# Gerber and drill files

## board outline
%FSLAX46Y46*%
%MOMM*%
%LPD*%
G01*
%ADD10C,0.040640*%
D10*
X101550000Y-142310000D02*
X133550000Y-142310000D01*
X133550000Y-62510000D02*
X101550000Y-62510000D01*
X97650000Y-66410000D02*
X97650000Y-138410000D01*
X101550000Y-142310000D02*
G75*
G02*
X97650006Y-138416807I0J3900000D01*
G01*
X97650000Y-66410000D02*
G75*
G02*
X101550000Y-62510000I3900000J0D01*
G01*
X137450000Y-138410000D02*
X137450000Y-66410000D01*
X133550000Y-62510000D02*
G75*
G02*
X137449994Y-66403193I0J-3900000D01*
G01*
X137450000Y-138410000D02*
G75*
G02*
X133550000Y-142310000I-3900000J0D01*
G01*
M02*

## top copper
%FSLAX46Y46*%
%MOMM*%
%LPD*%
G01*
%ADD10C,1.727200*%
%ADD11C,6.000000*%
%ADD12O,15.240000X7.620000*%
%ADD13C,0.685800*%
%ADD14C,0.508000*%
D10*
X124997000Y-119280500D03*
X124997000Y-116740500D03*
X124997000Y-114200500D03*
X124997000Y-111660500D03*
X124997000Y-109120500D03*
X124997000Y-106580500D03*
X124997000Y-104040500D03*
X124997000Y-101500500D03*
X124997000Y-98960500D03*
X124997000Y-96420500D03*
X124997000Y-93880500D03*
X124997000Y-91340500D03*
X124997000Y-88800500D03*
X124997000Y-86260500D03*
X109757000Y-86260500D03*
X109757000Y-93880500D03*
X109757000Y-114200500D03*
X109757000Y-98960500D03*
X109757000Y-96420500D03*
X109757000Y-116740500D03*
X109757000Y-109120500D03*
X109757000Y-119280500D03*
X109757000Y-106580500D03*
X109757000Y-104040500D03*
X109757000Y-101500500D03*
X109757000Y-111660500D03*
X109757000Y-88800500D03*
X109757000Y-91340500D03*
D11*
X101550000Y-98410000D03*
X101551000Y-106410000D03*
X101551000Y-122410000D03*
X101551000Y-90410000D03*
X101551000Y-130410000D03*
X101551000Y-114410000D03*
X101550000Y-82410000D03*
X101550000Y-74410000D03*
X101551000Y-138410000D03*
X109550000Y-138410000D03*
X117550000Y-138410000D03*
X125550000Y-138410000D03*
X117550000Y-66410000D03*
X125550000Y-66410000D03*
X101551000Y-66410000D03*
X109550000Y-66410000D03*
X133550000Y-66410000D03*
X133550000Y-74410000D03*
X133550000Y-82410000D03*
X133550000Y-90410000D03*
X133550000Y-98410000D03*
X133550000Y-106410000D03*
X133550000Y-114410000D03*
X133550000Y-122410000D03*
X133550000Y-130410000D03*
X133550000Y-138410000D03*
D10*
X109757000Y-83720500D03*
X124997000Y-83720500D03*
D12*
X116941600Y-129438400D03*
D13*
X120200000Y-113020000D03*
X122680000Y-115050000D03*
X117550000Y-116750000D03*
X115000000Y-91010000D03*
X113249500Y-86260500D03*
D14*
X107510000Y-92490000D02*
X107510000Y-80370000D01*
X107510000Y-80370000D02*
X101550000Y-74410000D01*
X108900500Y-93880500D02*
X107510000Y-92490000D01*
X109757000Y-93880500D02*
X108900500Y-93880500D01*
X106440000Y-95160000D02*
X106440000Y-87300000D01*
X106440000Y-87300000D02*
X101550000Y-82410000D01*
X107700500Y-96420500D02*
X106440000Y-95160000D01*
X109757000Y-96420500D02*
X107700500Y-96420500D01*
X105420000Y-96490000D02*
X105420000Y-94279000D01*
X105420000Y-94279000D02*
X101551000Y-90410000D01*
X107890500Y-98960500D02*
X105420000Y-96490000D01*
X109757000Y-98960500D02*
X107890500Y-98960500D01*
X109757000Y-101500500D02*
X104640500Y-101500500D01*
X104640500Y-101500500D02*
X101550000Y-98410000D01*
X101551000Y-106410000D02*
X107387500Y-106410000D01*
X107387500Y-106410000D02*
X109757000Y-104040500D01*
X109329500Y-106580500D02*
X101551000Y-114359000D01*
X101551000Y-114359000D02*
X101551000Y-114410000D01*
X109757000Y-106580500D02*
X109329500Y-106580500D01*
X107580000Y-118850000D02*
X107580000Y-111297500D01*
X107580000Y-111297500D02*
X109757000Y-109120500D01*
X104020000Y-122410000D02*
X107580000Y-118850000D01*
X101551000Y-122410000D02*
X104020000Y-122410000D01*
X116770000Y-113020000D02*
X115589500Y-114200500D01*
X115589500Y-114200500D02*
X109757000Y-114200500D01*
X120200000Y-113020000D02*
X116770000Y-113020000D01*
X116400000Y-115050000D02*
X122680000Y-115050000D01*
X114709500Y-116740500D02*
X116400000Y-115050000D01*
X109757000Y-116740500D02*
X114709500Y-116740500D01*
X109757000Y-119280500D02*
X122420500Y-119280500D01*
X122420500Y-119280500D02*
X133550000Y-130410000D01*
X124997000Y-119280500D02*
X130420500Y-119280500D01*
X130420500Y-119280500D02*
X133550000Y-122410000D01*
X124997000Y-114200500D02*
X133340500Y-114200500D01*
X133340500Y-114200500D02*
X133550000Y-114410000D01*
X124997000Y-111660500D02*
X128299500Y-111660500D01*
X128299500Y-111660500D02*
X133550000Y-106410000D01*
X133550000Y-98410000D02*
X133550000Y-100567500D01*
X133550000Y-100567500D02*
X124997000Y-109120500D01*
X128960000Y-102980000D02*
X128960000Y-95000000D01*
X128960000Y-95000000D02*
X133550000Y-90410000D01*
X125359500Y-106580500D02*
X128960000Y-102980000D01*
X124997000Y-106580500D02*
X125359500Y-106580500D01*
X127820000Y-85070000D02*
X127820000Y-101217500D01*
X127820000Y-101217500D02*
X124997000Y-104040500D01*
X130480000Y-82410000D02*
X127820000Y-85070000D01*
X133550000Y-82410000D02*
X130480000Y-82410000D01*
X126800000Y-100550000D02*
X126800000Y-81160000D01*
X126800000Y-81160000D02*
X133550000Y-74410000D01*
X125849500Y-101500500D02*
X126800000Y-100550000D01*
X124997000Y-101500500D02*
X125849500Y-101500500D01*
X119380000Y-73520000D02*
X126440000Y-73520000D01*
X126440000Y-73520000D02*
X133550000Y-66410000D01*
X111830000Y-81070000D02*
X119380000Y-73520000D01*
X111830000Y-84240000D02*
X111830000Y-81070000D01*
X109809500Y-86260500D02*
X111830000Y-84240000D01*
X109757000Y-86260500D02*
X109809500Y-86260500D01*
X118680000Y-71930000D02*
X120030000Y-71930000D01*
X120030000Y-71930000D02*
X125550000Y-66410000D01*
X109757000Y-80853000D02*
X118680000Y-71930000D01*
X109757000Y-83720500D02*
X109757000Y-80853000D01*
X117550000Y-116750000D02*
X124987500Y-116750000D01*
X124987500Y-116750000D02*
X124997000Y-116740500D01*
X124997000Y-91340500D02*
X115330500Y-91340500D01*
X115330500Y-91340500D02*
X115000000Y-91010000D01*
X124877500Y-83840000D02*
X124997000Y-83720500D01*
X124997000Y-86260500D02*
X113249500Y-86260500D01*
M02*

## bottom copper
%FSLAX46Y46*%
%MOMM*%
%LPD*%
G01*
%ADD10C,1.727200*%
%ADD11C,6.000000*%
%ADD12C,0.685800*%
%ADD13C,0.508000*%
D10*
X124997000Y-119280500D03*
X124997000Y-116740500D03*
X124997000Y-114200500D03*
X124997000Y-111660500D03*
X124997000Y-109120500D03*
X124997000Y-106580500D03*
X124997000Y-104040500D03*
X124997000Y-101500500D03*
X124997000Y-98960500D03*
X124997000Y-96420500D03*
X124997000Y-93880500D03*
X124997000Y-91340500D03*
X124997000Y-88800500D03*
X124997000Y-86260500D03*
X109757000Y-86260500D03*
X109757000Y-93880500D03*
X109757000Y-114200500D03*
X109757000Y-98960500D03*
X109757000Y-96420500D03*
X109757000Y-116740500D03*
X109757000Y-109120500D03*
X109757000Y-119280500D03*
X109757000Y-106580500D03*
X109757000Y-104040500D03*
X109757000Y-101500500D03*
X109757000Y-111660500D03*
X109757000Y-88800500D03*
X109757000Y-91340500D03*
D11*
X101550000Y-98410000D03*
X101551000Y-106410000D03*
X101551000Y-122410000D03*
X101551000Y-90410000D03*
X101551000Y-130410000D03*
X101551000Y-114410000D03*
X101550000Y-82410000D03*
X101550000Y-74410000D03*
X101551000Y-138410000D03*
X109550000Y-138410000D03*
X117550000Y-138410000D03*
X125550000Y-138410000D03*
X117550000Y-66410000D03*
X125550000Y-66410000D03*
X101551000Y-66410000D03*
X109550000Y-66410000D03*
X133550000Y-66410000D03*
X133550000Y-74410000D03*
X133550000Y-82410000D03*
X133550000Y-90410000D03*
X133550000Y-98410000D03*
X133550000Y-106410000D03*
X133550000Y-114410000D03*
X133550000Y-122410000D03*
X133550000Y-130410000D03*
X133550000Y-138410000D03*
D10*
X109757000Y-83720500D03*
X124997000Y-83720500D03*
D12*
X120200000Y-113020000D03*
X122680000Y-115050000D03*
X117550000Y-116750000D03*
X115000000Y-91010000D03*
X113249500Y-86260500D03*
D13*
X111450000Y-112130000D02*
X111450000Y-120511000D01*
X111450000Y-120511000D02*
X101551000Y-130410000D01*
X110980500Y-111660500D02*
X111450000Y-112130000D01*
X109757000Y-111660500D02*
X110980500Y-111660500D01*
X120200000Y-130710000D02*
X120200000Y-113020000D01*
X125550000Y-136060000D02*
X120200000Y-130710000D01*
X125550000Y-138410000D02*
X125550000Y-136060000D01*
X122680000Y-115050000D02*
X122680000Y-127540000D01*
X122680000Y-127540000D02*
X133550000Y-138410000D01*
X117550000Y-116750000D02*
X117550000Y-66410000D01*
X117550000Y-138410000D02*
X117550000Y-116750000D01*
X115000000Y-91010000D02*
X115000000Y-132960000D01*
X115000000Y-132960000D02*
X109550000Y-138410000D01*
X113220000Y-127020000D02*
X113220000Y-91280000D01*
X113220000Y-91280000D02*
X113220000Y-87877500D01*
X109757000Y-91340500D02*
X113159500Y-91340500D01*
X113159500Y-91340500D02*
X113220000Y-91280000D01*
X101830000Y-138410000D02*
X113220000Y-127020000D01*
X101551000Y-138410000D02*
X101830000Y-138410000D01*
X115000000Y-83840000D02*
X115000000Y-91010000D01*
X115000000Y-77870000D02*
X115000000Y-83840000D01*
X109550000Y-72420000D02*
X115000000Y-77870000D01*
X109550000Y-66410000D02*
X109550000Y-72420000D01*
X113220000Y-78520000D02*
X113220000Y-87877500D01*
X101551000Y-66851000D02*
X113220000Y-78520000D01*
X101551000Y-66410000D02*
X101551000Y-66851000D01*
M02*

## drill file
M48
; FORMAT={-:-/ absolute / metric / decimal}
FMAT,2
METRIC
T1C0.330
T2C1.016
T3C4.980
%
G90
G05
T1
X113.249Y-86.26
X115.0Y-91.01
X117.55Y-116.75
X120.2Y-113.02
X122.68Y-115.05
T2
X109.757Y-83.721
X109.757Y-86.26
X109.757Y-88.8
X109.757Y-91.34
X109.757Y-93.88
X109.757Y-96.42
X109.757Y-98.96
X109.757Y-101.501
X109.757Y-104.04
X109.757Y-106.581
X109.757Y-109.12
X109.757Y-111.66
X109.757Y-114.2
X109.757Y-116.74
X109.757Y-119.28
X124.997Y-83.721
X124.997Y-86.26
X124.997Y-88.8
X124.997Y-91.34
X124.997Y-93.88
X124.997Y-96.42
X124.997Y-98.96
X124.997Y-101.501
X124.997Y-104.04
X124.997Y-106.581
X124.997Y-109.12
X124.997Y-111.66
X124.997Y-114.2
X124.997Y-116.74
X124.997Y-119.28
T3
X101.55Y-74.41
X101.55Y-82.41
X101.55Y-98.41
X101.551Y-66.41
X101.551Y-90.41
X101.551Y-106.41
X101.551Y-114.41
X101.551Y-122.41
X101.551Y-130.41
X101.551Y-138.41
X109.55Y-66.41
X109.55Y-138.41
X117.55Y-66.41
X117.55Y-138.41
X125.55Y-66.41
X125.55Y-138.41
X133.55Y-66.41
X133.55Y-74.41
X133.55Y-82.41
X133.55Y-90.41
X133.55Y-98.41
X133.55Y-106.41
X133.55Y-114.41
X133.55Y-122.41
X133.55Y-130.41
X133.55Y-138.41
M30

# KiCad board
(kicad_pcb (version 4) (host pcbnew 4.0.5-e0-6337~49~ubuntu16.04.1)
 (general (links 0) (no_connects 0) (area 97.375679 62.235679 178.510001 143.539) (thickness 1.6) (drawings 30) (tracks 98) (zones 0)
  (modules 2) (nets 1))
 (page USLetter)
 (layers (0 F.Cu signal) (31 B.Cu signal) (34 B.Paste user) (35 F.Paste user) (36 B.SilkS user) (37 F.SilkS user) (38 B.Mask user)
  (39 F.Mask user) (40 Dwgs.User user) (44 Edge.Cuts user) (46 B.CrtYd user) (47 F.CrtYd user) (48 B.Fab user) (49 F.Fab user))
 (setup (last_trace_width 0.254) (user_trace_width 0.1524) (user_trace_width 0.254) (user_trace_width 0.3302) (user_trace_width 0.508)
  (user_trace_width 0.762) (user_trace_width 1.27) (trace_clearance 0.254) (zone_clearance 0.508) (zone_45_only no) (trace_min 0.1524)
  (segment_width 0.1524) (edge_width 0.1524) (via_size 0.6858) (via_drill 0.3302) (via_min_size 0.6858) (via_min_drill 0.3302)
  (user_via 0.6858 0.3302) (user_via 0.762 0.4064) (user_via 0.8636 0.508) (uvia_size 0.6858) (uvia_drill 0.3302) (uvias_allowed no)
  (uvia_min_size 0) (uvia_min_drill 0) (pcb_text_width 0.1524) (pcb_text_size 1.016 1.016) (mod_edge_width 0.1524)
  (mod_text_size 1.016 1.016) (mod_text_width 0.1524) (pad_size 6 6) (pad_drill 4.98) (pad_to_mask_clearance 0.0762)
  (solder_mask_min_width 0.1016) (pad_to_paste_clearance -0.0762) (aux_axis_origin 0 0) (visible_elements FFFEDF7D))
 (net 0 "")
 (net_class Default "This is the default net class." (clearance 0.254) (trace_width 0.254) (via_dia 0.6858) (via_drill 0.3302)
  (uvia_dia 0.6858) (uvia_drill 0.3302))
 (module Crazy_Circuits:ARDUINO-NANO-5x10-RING (layer F.Cu) (at 101.55 90.41)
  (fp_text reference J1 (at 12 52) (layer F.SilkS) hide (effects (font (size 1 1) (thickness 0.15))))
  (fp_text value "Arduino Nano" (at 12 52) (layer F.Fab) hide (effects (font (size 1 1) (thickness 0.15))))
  (fp_line (start 0 51.9) (end 32 51.9) (layer Edge.Cuts) (width 0.04064))
  (fp_line (start 32 -27.9) (end 0 -27.9) (layer Edge.Cuts) (width 0.04064))
  (fp_line (start -3.9 -24) (end -3.9 48) (layer Edge.Cuts) (width 0.04064))
  (fp_arc (start 0 48) (end 0 51.9) (angle 89.9) (layer Edge.Cuts) (width 0.04064))
  (fp_arc (start 0 -24) (end -3.9 -24) (angle 90) (layer Edge.Cuts) (width 0.04064))
  (fp_line (start 35.9 48) (end 35.9 -24) (layer Edge.Cuts) (width 0.04064))
  (fp_arc (start 32 -24) (end 32 -27.9) (angle 89.9) (layer Edge.Cuts) (width 0.04064))
  (fp_arc (start 32 48) (end 35.9 48) (angle 90) (layer Edge.Cuts) (width 0.04064))
  (pad D13 thru_hole circle (at 23.447 28.8705 180) (size 1.7272 1.7272) (drill 1.016) (layers *.Cu *.Mask F.SilkS))
  (pad 3V3 thru_hole circle (at 23.447 26.3305 180) (size 1.7272 1.7272) (drill 1.016) (layers *.Cu *.Mask F.SilkS))
  (pad REF thru_hole circle (at 23.447 23.7905 180) (size 1.7272 1.7272) (drill 1.016) (layers *.Cu *.Mask F.SilkS))
  (pad A0 thru_hole circle (at 23.447 21.2505 180) (size 1.7272 1.7272) (drill 1.016) (layers *.Cu *.Mask F.SilkS))
  (pad A1 thru_hole circle (at 23.447 18.7105 180) (size 1.7272 1.7272) (drill 1.016) (layers *.Cu *.Mask F.SilkS))
  (pad A2 thru_hole circle (at 23.447 16.1705 180) (size 1.7272 1.7272) (drill 1.016) (layers *.Cu *.Mask F.SilkS))
  (pad A3 thru_hole circle (at 23.447 13.6305 180) (size 1.7272 1.7272) (drill 1.016) (layers *.Cu *.Mask F.SilkS))
  (pad A4 thru_hole circle (at 23.447 11.0905 180) (size 1.7272 1.7272) (drill 1.016) (layers *.Cu *.Mask F.SilkS))
  (pad A5 thru_hole circle (at 23.447 8.5505 180) (size 1.7272 1.7272) (drill 1.016) (layers *.Cu *.Mask F.SilkS))
  (pad A6 thru_hole circle (at 23.447 6.0105 180) (size 1.7272 1.7272) (drill 1.016) (layers *.Cu *.Mask F.SilkS))
  (pad A7 thru_hole circle (at 23.447 3.4705 180) (size 1.7272 1.7272) (drill 1.016) (layers *.Cu *.Mask F.SilkS))
  (pad 5V thru_hole circle (at 23.447 0.9305 180) (size 1.7272 1.7272) (drill 1.016) (layers *.Cu *.Mask F.SilkS))
  (pad RST thru_hole circle (at 23.447 -1.6095 180) (size 1.7272 1.7272) (drill 1.016) (layers *.Cu *.Mask F.SilkS))
  (pad GND thru_hole circle (at 23.447 -4.1495 180) (size 1.7272 1.7272) (drill 1.016) (layers *.Cu *.Mask F.SilkS))
  (pad D0RX thru_hole circle (at 8.207 -4.1495 180) (size 1.7272 1.7272) (drill 1.016) (layers *.Cu *.Mask F.SilkS))
  (pad D2 thru_hole circle (at 8.207 3.4705 180) (size 1.7272 1.7272) (drill 1.016) (layers *.Cu *.Mask F.SilkS))
  (pad D10 thru_hole circle (at 8.207 23.7905 180) (size 1.7272 1.7272) (drill 1.016) (layers *.Cu *.Mask F.SilkS))
  (pad D4 thru_hole circle (at 8.207 8.5505 180) (size 1.7272 1.7272) (drill 1.016) (layers *.Cu *.Mask F.SilkS))
  (pad D3 thru_hole circle (at 8.207 6.0105 180) (size 1.7272 1.7272) (drill 1.016) (layers *.Cu *.Mask F.SilkS))
  (pad D11 thru_hole circle (at 8.207 26.3305 180) (size 1.7272 1.7272) (drill 1.016) (layers *.Cu *.Mask F.SilkS))
  (pad D8 thru_hole circle (at 8.207 18.7105 180) (size 1.7272 1.7272) (drill 1.016) (layers *.Cu *.Mask F.SilkS))
  (pad D12 thru_hole circle (at 8.207 28.8705 180) (size 1.7272 1.7272) (drill 1.016) (layers *.Cu *.Mask F.SilkS))
  (pad D7 thru_hole circle (at 8.207 16.1705 180) (size 1.7272 1.7272) (drill 1.016) (layers *.Cu *.Mask F.SilkS))
  (pad D6 thru_hole circle (at 8.207 13.6305 180) (size 1.7272 1.7272) (drill 1.016) (layers *.Cu *.Mask F.SilkS))
  (pad D5 thru_hole circle (at 8.207 11.0905 180) (size 1.7272 1.7272) (drill 1.016) (layers *.Cu *.Mask F.SilkS))
  (pad D9 thru_hole circle (at 8.207 21.2505 180) (size 1.7272 1.7272) (drill 1.016) (layers *.Cu *.Mask F.SilkS))
  (pad RST thru_hole circle (at 8.207 -1.6095 180) (size 1.7272 1.7272) (drill 1.016) (layers *.Cu *.Mask F.SilkS))
  (pad GND thru_hole circle (at 8.207 0.9305 180) (size 1.7272 1.7272) (drill 1.016) (layers *.Cu *.Mask F.SilkS))
  (pad D5 thru_hole circle (at 0 8 90) (size 6 6) (drill 4.98) (layers *.Cu *.Mask))
  (pad D6 thru_hole circle (at 0.001 16 90) (size 6 6) (drill 4.98) (layers *.Cu *.Mask))
  (pad D8 thru_hole circle (at 0.001 32 90) (size 6 6) (drill 4.98) (layers *.Cu *.Mask))
  (pad D4 thru_hole circle (at 0.001 0 90) (size 6 6) (drill 4.98) (layers *.Cu *.Mask))
  (pad D9 thru_hole circle (at 0.001 40 90) (size 6 6) (drill 4.98) (layers *.Cu *.Mask))
  (pad D7 thru_hole circle (at 0.001 24 90) (size 6 6) (drill 4.98) (layers *.Cu *.Mask))
  (pad D3 thru_hole circle (at 0 -8 90) (size 6 6) (drill 4.98) (layers *.Cu *.Mask))
  (pad D2 thru_hole circle (at 0 -16 90) (size 6 6) (drill 4.98) (layers *.Cu *.Mask))
  (pad GND thru_hole circle (at 0.001 48 90) (size 6 6) (drill 4.98) (layers *.Cu *.Mask))
  (pad 5V thru_hole circle (at 8 48 90) (size 6 6) (drill 4.98) (layers *.Cu *.Mask))
  (pad 3.3V thru_hole circle (at 16 48 90) (size 6 6) (drill 4.98) (layers *.Cu *.Mask))
  (pad D10 thru_hole circle (at 24 48 90) (size 6 6) (drill 4.98) (layers *.Cu *.Mask))
  (pad 3.3V thru_hole circle (at 16 -24 90) (size 6 6) (drill 4.98) (layers *.Cu *.Mask))
  (pad D1TX thru_hole circle (at 24 -24 90) (size 6 6) (drill 4.98) (layers *.Cu *.Mask))
  (pad GND thru_hole circle (at 0.001 -24 90) (size 6 6) (drill 4.98) (layers *.Cu *.Mask))
  (pad 5V thru_hole circle (at 8 -24 90) (size 6 6) (drill 4.98) (layers *.Cu *.Mask))
  (pad D0RX thru_hole circle (at 32 -24 90) (size 6 6) (drill 4.98) (layers *.Cu *.Mask))
  (pad A4 thru_hole circle (at 32 -16 90) (size 6 6) (drill 4.98) (layers *.Cu *.Mask))
  (pad A3 thru_hole circle (at 32 -8 90) (size 6 6) (drill 4.98) (layers *.Cu *.Mask))
  (pad A2 thru_hole circle (at 32 0 90) (size 6 6) (drill 4.98) (layers *.Cu *.Mask))
  (pad A1 thru_hole circle (at 32 8 90) (size 6 6) (drill 4.98) (layers *.Cu *.Mask))
  (pad A0 thru_hole circle (at 32 16 90) (size 6 6) (drill 4.98) (layers *.Cu *.Mask))
  (pad AREF thru_hole circle (at 32 24 90) (size 6 6) (drill 4.98) (layers *.Cu *.Mask))
  (pad D13 thru_hole circle (at 32 32 90) (size 6 6) (drill 4.98) (layers *.Cu *.Mask))
  (pad D12 thru_hole circle (at 32 40 90) (size 6 6) (drill 4.98) (layers *.Cu *.Mask))
  (pad D11 thru_hole circle (at 32 48 90) (size 6 6) (drill 4.98) (layers *.Cu *.Mask))
  (pad D1TX thru_hole circle (at 8.207 -6.6895 180) (size 1.7272 1.7272) (drill 1.016) (layers *.Cu *.Mask F.SilkS))
  (pad VIN thru_hole circle (at 23.447 -6.6895 180) (size 1.7272 1.7272) (drill 1.016) (layers *.Cu *.Mask F.SilkS)))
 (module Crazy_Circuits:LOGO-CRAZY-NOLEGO (layer F.Cu) (at 116.9416 133.3754)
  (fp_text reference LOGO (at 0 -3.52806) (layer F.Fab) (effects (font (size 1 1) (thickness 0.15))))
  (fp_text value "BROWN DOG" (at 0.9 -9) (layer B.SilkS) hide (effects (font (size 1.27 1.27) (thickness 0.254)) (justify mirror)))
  (pad BG smd oval (at 0 -3.937) (size 15.24 7.62) (layers F.Cu)))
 (segment (start 107.51 92.49) (end 107.51 80.37) (width 0.508) (layer F.Cu) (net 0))
 (segment (start 107.51 80.37) (end 101.55 74.41) (width 0.508) (layer F.Cu) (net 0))
 (segment (start 108.9005 93.8805) (end 107.51 92.49) (width 0.508) (layer F.Cu) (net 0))
 (segment (start 109.757 93.8805) (end 108.9005 93.8805) (width 0.508) (layer F.Cu) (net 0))
 (segment (start 106.44 95.16) (end 106.44 87.3) (width 0.508) (layer F.Cu) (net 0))
 (segment (start 106.44 87.3) (end 101.55 82.41) (width 0.508) (layer F.Cu) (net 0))
 (segment (start 107.7005 96.4205) (end 106.44 95.16) (width 0.508) (layer F.Cu) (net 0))
 (segment (start 109.757 96.4205) (end 107.7005 96.4205) (width 0.508) (layer F.Cu) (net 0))
 (segment (start 105.42 96.49) (end 105.42 94.279) (width 0.508) (layer F.Cu) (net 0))
 (segment (start 105.42 94.279) (end 101.551 90.41) (width 0.508) (layer F.Cu) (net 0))
 (segment (start 107.8905 98.9605) (end 105.42 96.49) (width 0.508) (layer F.Cu) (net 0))
 (segment (start 109.757 98.9605) (end 107.8905 98.9605) (width 0.508) (layer F.Cu) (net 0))
 (segment (start 109.757 101.5005) (end 104.6405 101.5005) (width 0.508) (layer F.Cu) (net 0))
 (segment (start 104.6405 101.5005) (end 101.55 98.41) (width 0.508) (layer F.Cu) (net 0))
 (segment (start 101.551 106.41) (end 107.3875 106.41) (width 0.508) (layer F.Cu) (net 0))
 (segment (start 107.3875 106.41) (end 109.757 104.0405) (width 0.508) (layer F.Cu) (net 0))
 (segment (start 109.3295 106.5805) (end 101.551 114.359) (width 0.508) (layer F.Cu) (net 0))
 (segment (start 101.551 114.359) (end 101.551 114.41) (width 0.508) (layer F.Cu) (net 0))
 (segment (start 109.757 106.5805) (end 109.3295 106.5805) (width 0.508) (layer F.Cu) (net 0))
 (segment (start 107.58 118.85) (end 107.58 111.2975) (width 0.508) (layer F.Cu) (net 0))
 (segment (start 107.58 111.2975) (end 109.757 109.1205) (width 0.508) (layer F.Cu) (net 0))
 (segment (start 104.02 122.41) (end 107.58 118.85) (width 0.508) (layer F.Cu) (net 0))
 (segment (start 101.551 122.41) (end 104.02 122.41) (width 0.508) (layer F.Cu) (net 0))
 (segment (start 111.45 112.13) (end 111.45 120.511) (width 0.508) (layer B.Cu) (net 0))
 (segment (start 111.45 120.511) (end 101.551 130.41) (width 0.508) (layer B.Cu) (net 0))
 (segment (start 110.9805 111.6605) (end 111.45 112.13) (width 0.508) (layer B.Cu) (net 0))
 (segment (start 109.757 111.6605) (end 110.9805 111.6605) (width 0.508) (layer B.Cu) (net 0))
 (segment (start 116.77 113.02) (end 115.5895 114.2005) (width 0.508) (layer F.Cu) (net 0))
 (segment (start 115.5895 114.2005) (end 109.757 114.2005) (width 0.508) (layer F.Cu) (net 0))
 (segment (start 120.2 113.02) (end 116.77 113.02) (width 0.508) (layer F.Cu) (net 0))
 (segment (start 120.2 130.71) (end 120.2 113.02) (width 0.508) (layer B.Cu) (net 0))
 (via (at 120.2 113.02) (size 0.6858) (drill 0.3302) (layers F.Cu B.Cu) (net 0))
 (segment (start 125.55 136.06) (end 120.2 130.71) (width 0.508) (layer B.Cu) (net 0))
 (segment (start 125.55 138.41) (end 125.55 136.06) (width 0.508) (layer B.Cu) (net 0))
 (segment (start 122.68 115.05) (end 122.68 127.54) (width 0.508) (layer B.Cu) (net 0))
 (segment (start 122.68 127.54) (end 133.55 138.41) (width 0.508) (layer B.Cu) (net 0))
 (via (at 122.68 115.05) (size 0.6858) (drill 0.3302) (layers F.Cu B.Cu) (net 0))
 (segment (start 116.4 115.05) (end 122.68 115.05) (width 0.508) (layer F.Cu) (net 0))
 (segment (start 114.7095 116.7405) (end 116.4 115.05) (width 0.508) (layer F.Cu) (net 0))
 (segment (start 109.757 116.7405) (end 114.7095 116.7405) (width 0.508) (layer F.Cu) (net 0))
 (segment (start 109.757 119.2805) (end 122.4205 119.2805) (width 0.508) (layer F.Cu) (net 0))
 (segment (start 122.4205 119.2805) (end 133.55 130.41) (width 0.508) (layer F.Cu) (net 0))
 (segment (start 124.997 119.2805) (end 130.4205 119.2805) (width 0.508) (layer F.Cu) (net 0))
 (segment (start 130.4205 119.2805) (end 133.55 122.41) (width 0.508) (layer F.Cu) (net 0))
 (segment (start 124.997 114.2005) (end 133.3405 114.2005) (width 0.508) (layer F.Cu) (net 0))
 (segment (start 133.3405 114.2005) (end 133.55 114.41) (width 0.508) (layer F.Cu) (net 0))
 (segment (start 124.997 111.6605) (end 128.2995 111.6605) (width 0.508) (layer F.Cu) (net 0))
 (segment (start 128.2995 111.6605) (end 133.55 106.41) (width 0.508) (layer F.Cu) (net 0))
 (segment (start 133.55 98.41) (end 133.55 100.5675) (width 0.508) (layer F.Cu) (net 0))
 (segment (start 133.55 100.5675) (end 124.997 109.1205) (width 0.508) (layer F.Cu) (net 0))
 (segment (start 128.96 102.98) (end 128.96 95) (width 0.508) (layer F.Cu) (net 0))
 (segment (start 128.96 95) (end 133.55 90.41) (width 0.508) (layer F.Cu) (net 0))
 (segment (start 125.3595 106.5805) (end 128.96 102.98) (width 0.508) (layer F.Cu) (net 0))
 (segment (start 124.997 106.5805) (end 125.3595 106.5805) (width 0.508) (layer F.Cu) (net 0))
 (segment (start 127.82 85.07) (end 127.82 101.2175) (width 0.508) (layer F.Cu) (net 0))
 (segment (start 127.82 101.2175) (end 124.997 104.0405) (width 0.508) (layer F.Cu) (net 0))
 (segment (start 130.48 82.41) (end 127.82 85.07) (width 0.508) (layer F.Cu) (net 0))
 (segment (start 133.55 82.41) (end 130.48 82.41) (width 0.508) (layer F.Cu) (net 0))
 (segment (start 126.8 100.55) (end 126.8 81.16) (width 0.508) (layer F.Cu) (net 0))
 (segment (start 126.8 81.16) (end 133.55 74.41) (width 0.508) (layer F.Cu) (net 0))
 (segment (start 125.8495 101.5005) (end 126.8 100.55) (width 0.508) (layer F.Cu) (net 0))
 (segment (start 124.997 101.5005) (end 125.8495 101.5005) (width 0.508) (layer F.Cu) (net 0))
 (segment (start 119.38 73.52) (end 126.44 73.52) (width 0.508) (layer F.Cu) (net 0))
 (segment (start 126.44 73.52) (end 133.55 66.41) (width 0.508) (layer F.Cu) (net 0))
 (segment (start 111.83 81.07) (end 119.38 73.52) (width 0.508) (layer F.Cu) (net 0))
 (segment (start 111.83 84.24) (end 111.83 81.07) (width 0.508) (layer F.Cu) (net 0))
 (segment (start 109.8095 86.2605) (end 111.83 84.24) (width 0.508) (layer F.Cu) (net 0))
 (segment (start 109.757 86.2605) (end 109.8095 86.2605) (width 0.508) (layer F.Cu) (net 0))
 (segment (start 118.68 71.93) (end 120.03 71.93) (width 0.508) (layer F.Cu) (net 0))
 (segment (start 120.03 71.93) (end 125.55 66.41) (width 0.508) (layer F.Cu) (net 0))
 (segment (start 109.757 80.853) (end 118.68 71.93) (width 0.508) (layer F.Cu) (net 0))
 (segment (start 109.757 83.7205) (end 109.757 80.853) (width 0.508) (layer F.Cu) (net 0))
 (segment (start 117.55 116.75) (end 117.55 66.41) (width 0.508) (layer B.Cu) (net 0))
 (segment (start 117.55 116.75) (end 124.9875 116.75) (width 0.508) (layer F.Cu) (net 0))
 (segment (start 124.9875 116.75) (end 124.997 116.7405) (width 0.508) (layer F.Cu) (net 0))
 (via (at 117.55 116.75) (size 0.6858) (drill 0.3302) (layers F.Cu B.Cu) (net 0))
 (segment (start 117.55 138.41) (end 117.55 116.75) (width 0.508) (layer B.Cu) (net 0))
 (segment (start 115 91.01) (end 115 132.96) (width 0.508) (layer B.Cu) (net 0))
 (segment (start 115 132.96) (end 109.55 138.41) (width 0.508) (layer B.Cu) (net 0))
 (segment (start 113.22 127.02) (end 113.22 91.28) (width 0.508) (layer B.Cu) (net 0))
 (segment (start 113.22 91.28) (end 113.22 87.8775) (width 0.508) (layer B.Cu) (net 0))
 (segment (start 109.757 91.3405) (end 113.1595 91.3405) (width 0.508) (layer B.Cu) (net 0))
 (segment (start 113.1595 91.3405) (end 113.22 91.28) (width 0.508) (layer B.Cu) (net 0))
 (segment (start 101.83 138.41) (end 113.22 127.02) (width 0.508) (layer B.Cu) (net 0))
 (segment (start 101.551 138.41) (end 101.83 138.41) (width 0.508) (layer B.Cu) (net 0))
 (segment (start 124.997 91.3405) (end 115.3305 91.3405) (width 0.508) (layer F.Cu) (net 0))
 (segment (start 115.3305 91.3405) (end 115 91.01) (width 0.508) (layer F.Cu) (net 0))
 (via (at 115 91.01) (size 0.6858) (drill 0.3302) (layers F.Cu B.Cu) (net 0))
 (segment (start 115 83.84) (end 115 91.01) (width 0.508) (layer B.Cu) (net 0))
 (segment (start 124.8775 83.84) (end 124.997 83.7205) (width 0.508) (layer F.Cu) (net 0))
 (segment (start 115 77.87) (end 115 83.84) (width 0.508) (layer B.Cu) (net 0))
 (segment (start 109.55 72.42) (end 115 77.87) (width 0.508) (layer B.Cu) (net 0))
 (segment (start 109.55 66.41) (end 109.55 72.42) (width 0.508) (layer B.Cu) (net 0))
 (via (at 113.2495 86.2605) (size 0.6858) (drill 0.3302) (layers F.Cu B.Cu) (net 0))
 (segment (start 124.997 86.2605) (end 113.2495 86.2605) (width 0.508) (layer F.Cu) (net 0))
 (segment (start 113.22 78.52) (end 113.22 87.8775) (width 0.508) (layer B.Cu) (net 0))
 (segment (start 101.551 66.851) (end 113.22 78.52) (width 0.508) (layer B.Cu) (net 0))
 (segment (start 101.551 66.41) (end 101.551 66.851) (width 0.508) (layer B.Cu) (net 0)))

